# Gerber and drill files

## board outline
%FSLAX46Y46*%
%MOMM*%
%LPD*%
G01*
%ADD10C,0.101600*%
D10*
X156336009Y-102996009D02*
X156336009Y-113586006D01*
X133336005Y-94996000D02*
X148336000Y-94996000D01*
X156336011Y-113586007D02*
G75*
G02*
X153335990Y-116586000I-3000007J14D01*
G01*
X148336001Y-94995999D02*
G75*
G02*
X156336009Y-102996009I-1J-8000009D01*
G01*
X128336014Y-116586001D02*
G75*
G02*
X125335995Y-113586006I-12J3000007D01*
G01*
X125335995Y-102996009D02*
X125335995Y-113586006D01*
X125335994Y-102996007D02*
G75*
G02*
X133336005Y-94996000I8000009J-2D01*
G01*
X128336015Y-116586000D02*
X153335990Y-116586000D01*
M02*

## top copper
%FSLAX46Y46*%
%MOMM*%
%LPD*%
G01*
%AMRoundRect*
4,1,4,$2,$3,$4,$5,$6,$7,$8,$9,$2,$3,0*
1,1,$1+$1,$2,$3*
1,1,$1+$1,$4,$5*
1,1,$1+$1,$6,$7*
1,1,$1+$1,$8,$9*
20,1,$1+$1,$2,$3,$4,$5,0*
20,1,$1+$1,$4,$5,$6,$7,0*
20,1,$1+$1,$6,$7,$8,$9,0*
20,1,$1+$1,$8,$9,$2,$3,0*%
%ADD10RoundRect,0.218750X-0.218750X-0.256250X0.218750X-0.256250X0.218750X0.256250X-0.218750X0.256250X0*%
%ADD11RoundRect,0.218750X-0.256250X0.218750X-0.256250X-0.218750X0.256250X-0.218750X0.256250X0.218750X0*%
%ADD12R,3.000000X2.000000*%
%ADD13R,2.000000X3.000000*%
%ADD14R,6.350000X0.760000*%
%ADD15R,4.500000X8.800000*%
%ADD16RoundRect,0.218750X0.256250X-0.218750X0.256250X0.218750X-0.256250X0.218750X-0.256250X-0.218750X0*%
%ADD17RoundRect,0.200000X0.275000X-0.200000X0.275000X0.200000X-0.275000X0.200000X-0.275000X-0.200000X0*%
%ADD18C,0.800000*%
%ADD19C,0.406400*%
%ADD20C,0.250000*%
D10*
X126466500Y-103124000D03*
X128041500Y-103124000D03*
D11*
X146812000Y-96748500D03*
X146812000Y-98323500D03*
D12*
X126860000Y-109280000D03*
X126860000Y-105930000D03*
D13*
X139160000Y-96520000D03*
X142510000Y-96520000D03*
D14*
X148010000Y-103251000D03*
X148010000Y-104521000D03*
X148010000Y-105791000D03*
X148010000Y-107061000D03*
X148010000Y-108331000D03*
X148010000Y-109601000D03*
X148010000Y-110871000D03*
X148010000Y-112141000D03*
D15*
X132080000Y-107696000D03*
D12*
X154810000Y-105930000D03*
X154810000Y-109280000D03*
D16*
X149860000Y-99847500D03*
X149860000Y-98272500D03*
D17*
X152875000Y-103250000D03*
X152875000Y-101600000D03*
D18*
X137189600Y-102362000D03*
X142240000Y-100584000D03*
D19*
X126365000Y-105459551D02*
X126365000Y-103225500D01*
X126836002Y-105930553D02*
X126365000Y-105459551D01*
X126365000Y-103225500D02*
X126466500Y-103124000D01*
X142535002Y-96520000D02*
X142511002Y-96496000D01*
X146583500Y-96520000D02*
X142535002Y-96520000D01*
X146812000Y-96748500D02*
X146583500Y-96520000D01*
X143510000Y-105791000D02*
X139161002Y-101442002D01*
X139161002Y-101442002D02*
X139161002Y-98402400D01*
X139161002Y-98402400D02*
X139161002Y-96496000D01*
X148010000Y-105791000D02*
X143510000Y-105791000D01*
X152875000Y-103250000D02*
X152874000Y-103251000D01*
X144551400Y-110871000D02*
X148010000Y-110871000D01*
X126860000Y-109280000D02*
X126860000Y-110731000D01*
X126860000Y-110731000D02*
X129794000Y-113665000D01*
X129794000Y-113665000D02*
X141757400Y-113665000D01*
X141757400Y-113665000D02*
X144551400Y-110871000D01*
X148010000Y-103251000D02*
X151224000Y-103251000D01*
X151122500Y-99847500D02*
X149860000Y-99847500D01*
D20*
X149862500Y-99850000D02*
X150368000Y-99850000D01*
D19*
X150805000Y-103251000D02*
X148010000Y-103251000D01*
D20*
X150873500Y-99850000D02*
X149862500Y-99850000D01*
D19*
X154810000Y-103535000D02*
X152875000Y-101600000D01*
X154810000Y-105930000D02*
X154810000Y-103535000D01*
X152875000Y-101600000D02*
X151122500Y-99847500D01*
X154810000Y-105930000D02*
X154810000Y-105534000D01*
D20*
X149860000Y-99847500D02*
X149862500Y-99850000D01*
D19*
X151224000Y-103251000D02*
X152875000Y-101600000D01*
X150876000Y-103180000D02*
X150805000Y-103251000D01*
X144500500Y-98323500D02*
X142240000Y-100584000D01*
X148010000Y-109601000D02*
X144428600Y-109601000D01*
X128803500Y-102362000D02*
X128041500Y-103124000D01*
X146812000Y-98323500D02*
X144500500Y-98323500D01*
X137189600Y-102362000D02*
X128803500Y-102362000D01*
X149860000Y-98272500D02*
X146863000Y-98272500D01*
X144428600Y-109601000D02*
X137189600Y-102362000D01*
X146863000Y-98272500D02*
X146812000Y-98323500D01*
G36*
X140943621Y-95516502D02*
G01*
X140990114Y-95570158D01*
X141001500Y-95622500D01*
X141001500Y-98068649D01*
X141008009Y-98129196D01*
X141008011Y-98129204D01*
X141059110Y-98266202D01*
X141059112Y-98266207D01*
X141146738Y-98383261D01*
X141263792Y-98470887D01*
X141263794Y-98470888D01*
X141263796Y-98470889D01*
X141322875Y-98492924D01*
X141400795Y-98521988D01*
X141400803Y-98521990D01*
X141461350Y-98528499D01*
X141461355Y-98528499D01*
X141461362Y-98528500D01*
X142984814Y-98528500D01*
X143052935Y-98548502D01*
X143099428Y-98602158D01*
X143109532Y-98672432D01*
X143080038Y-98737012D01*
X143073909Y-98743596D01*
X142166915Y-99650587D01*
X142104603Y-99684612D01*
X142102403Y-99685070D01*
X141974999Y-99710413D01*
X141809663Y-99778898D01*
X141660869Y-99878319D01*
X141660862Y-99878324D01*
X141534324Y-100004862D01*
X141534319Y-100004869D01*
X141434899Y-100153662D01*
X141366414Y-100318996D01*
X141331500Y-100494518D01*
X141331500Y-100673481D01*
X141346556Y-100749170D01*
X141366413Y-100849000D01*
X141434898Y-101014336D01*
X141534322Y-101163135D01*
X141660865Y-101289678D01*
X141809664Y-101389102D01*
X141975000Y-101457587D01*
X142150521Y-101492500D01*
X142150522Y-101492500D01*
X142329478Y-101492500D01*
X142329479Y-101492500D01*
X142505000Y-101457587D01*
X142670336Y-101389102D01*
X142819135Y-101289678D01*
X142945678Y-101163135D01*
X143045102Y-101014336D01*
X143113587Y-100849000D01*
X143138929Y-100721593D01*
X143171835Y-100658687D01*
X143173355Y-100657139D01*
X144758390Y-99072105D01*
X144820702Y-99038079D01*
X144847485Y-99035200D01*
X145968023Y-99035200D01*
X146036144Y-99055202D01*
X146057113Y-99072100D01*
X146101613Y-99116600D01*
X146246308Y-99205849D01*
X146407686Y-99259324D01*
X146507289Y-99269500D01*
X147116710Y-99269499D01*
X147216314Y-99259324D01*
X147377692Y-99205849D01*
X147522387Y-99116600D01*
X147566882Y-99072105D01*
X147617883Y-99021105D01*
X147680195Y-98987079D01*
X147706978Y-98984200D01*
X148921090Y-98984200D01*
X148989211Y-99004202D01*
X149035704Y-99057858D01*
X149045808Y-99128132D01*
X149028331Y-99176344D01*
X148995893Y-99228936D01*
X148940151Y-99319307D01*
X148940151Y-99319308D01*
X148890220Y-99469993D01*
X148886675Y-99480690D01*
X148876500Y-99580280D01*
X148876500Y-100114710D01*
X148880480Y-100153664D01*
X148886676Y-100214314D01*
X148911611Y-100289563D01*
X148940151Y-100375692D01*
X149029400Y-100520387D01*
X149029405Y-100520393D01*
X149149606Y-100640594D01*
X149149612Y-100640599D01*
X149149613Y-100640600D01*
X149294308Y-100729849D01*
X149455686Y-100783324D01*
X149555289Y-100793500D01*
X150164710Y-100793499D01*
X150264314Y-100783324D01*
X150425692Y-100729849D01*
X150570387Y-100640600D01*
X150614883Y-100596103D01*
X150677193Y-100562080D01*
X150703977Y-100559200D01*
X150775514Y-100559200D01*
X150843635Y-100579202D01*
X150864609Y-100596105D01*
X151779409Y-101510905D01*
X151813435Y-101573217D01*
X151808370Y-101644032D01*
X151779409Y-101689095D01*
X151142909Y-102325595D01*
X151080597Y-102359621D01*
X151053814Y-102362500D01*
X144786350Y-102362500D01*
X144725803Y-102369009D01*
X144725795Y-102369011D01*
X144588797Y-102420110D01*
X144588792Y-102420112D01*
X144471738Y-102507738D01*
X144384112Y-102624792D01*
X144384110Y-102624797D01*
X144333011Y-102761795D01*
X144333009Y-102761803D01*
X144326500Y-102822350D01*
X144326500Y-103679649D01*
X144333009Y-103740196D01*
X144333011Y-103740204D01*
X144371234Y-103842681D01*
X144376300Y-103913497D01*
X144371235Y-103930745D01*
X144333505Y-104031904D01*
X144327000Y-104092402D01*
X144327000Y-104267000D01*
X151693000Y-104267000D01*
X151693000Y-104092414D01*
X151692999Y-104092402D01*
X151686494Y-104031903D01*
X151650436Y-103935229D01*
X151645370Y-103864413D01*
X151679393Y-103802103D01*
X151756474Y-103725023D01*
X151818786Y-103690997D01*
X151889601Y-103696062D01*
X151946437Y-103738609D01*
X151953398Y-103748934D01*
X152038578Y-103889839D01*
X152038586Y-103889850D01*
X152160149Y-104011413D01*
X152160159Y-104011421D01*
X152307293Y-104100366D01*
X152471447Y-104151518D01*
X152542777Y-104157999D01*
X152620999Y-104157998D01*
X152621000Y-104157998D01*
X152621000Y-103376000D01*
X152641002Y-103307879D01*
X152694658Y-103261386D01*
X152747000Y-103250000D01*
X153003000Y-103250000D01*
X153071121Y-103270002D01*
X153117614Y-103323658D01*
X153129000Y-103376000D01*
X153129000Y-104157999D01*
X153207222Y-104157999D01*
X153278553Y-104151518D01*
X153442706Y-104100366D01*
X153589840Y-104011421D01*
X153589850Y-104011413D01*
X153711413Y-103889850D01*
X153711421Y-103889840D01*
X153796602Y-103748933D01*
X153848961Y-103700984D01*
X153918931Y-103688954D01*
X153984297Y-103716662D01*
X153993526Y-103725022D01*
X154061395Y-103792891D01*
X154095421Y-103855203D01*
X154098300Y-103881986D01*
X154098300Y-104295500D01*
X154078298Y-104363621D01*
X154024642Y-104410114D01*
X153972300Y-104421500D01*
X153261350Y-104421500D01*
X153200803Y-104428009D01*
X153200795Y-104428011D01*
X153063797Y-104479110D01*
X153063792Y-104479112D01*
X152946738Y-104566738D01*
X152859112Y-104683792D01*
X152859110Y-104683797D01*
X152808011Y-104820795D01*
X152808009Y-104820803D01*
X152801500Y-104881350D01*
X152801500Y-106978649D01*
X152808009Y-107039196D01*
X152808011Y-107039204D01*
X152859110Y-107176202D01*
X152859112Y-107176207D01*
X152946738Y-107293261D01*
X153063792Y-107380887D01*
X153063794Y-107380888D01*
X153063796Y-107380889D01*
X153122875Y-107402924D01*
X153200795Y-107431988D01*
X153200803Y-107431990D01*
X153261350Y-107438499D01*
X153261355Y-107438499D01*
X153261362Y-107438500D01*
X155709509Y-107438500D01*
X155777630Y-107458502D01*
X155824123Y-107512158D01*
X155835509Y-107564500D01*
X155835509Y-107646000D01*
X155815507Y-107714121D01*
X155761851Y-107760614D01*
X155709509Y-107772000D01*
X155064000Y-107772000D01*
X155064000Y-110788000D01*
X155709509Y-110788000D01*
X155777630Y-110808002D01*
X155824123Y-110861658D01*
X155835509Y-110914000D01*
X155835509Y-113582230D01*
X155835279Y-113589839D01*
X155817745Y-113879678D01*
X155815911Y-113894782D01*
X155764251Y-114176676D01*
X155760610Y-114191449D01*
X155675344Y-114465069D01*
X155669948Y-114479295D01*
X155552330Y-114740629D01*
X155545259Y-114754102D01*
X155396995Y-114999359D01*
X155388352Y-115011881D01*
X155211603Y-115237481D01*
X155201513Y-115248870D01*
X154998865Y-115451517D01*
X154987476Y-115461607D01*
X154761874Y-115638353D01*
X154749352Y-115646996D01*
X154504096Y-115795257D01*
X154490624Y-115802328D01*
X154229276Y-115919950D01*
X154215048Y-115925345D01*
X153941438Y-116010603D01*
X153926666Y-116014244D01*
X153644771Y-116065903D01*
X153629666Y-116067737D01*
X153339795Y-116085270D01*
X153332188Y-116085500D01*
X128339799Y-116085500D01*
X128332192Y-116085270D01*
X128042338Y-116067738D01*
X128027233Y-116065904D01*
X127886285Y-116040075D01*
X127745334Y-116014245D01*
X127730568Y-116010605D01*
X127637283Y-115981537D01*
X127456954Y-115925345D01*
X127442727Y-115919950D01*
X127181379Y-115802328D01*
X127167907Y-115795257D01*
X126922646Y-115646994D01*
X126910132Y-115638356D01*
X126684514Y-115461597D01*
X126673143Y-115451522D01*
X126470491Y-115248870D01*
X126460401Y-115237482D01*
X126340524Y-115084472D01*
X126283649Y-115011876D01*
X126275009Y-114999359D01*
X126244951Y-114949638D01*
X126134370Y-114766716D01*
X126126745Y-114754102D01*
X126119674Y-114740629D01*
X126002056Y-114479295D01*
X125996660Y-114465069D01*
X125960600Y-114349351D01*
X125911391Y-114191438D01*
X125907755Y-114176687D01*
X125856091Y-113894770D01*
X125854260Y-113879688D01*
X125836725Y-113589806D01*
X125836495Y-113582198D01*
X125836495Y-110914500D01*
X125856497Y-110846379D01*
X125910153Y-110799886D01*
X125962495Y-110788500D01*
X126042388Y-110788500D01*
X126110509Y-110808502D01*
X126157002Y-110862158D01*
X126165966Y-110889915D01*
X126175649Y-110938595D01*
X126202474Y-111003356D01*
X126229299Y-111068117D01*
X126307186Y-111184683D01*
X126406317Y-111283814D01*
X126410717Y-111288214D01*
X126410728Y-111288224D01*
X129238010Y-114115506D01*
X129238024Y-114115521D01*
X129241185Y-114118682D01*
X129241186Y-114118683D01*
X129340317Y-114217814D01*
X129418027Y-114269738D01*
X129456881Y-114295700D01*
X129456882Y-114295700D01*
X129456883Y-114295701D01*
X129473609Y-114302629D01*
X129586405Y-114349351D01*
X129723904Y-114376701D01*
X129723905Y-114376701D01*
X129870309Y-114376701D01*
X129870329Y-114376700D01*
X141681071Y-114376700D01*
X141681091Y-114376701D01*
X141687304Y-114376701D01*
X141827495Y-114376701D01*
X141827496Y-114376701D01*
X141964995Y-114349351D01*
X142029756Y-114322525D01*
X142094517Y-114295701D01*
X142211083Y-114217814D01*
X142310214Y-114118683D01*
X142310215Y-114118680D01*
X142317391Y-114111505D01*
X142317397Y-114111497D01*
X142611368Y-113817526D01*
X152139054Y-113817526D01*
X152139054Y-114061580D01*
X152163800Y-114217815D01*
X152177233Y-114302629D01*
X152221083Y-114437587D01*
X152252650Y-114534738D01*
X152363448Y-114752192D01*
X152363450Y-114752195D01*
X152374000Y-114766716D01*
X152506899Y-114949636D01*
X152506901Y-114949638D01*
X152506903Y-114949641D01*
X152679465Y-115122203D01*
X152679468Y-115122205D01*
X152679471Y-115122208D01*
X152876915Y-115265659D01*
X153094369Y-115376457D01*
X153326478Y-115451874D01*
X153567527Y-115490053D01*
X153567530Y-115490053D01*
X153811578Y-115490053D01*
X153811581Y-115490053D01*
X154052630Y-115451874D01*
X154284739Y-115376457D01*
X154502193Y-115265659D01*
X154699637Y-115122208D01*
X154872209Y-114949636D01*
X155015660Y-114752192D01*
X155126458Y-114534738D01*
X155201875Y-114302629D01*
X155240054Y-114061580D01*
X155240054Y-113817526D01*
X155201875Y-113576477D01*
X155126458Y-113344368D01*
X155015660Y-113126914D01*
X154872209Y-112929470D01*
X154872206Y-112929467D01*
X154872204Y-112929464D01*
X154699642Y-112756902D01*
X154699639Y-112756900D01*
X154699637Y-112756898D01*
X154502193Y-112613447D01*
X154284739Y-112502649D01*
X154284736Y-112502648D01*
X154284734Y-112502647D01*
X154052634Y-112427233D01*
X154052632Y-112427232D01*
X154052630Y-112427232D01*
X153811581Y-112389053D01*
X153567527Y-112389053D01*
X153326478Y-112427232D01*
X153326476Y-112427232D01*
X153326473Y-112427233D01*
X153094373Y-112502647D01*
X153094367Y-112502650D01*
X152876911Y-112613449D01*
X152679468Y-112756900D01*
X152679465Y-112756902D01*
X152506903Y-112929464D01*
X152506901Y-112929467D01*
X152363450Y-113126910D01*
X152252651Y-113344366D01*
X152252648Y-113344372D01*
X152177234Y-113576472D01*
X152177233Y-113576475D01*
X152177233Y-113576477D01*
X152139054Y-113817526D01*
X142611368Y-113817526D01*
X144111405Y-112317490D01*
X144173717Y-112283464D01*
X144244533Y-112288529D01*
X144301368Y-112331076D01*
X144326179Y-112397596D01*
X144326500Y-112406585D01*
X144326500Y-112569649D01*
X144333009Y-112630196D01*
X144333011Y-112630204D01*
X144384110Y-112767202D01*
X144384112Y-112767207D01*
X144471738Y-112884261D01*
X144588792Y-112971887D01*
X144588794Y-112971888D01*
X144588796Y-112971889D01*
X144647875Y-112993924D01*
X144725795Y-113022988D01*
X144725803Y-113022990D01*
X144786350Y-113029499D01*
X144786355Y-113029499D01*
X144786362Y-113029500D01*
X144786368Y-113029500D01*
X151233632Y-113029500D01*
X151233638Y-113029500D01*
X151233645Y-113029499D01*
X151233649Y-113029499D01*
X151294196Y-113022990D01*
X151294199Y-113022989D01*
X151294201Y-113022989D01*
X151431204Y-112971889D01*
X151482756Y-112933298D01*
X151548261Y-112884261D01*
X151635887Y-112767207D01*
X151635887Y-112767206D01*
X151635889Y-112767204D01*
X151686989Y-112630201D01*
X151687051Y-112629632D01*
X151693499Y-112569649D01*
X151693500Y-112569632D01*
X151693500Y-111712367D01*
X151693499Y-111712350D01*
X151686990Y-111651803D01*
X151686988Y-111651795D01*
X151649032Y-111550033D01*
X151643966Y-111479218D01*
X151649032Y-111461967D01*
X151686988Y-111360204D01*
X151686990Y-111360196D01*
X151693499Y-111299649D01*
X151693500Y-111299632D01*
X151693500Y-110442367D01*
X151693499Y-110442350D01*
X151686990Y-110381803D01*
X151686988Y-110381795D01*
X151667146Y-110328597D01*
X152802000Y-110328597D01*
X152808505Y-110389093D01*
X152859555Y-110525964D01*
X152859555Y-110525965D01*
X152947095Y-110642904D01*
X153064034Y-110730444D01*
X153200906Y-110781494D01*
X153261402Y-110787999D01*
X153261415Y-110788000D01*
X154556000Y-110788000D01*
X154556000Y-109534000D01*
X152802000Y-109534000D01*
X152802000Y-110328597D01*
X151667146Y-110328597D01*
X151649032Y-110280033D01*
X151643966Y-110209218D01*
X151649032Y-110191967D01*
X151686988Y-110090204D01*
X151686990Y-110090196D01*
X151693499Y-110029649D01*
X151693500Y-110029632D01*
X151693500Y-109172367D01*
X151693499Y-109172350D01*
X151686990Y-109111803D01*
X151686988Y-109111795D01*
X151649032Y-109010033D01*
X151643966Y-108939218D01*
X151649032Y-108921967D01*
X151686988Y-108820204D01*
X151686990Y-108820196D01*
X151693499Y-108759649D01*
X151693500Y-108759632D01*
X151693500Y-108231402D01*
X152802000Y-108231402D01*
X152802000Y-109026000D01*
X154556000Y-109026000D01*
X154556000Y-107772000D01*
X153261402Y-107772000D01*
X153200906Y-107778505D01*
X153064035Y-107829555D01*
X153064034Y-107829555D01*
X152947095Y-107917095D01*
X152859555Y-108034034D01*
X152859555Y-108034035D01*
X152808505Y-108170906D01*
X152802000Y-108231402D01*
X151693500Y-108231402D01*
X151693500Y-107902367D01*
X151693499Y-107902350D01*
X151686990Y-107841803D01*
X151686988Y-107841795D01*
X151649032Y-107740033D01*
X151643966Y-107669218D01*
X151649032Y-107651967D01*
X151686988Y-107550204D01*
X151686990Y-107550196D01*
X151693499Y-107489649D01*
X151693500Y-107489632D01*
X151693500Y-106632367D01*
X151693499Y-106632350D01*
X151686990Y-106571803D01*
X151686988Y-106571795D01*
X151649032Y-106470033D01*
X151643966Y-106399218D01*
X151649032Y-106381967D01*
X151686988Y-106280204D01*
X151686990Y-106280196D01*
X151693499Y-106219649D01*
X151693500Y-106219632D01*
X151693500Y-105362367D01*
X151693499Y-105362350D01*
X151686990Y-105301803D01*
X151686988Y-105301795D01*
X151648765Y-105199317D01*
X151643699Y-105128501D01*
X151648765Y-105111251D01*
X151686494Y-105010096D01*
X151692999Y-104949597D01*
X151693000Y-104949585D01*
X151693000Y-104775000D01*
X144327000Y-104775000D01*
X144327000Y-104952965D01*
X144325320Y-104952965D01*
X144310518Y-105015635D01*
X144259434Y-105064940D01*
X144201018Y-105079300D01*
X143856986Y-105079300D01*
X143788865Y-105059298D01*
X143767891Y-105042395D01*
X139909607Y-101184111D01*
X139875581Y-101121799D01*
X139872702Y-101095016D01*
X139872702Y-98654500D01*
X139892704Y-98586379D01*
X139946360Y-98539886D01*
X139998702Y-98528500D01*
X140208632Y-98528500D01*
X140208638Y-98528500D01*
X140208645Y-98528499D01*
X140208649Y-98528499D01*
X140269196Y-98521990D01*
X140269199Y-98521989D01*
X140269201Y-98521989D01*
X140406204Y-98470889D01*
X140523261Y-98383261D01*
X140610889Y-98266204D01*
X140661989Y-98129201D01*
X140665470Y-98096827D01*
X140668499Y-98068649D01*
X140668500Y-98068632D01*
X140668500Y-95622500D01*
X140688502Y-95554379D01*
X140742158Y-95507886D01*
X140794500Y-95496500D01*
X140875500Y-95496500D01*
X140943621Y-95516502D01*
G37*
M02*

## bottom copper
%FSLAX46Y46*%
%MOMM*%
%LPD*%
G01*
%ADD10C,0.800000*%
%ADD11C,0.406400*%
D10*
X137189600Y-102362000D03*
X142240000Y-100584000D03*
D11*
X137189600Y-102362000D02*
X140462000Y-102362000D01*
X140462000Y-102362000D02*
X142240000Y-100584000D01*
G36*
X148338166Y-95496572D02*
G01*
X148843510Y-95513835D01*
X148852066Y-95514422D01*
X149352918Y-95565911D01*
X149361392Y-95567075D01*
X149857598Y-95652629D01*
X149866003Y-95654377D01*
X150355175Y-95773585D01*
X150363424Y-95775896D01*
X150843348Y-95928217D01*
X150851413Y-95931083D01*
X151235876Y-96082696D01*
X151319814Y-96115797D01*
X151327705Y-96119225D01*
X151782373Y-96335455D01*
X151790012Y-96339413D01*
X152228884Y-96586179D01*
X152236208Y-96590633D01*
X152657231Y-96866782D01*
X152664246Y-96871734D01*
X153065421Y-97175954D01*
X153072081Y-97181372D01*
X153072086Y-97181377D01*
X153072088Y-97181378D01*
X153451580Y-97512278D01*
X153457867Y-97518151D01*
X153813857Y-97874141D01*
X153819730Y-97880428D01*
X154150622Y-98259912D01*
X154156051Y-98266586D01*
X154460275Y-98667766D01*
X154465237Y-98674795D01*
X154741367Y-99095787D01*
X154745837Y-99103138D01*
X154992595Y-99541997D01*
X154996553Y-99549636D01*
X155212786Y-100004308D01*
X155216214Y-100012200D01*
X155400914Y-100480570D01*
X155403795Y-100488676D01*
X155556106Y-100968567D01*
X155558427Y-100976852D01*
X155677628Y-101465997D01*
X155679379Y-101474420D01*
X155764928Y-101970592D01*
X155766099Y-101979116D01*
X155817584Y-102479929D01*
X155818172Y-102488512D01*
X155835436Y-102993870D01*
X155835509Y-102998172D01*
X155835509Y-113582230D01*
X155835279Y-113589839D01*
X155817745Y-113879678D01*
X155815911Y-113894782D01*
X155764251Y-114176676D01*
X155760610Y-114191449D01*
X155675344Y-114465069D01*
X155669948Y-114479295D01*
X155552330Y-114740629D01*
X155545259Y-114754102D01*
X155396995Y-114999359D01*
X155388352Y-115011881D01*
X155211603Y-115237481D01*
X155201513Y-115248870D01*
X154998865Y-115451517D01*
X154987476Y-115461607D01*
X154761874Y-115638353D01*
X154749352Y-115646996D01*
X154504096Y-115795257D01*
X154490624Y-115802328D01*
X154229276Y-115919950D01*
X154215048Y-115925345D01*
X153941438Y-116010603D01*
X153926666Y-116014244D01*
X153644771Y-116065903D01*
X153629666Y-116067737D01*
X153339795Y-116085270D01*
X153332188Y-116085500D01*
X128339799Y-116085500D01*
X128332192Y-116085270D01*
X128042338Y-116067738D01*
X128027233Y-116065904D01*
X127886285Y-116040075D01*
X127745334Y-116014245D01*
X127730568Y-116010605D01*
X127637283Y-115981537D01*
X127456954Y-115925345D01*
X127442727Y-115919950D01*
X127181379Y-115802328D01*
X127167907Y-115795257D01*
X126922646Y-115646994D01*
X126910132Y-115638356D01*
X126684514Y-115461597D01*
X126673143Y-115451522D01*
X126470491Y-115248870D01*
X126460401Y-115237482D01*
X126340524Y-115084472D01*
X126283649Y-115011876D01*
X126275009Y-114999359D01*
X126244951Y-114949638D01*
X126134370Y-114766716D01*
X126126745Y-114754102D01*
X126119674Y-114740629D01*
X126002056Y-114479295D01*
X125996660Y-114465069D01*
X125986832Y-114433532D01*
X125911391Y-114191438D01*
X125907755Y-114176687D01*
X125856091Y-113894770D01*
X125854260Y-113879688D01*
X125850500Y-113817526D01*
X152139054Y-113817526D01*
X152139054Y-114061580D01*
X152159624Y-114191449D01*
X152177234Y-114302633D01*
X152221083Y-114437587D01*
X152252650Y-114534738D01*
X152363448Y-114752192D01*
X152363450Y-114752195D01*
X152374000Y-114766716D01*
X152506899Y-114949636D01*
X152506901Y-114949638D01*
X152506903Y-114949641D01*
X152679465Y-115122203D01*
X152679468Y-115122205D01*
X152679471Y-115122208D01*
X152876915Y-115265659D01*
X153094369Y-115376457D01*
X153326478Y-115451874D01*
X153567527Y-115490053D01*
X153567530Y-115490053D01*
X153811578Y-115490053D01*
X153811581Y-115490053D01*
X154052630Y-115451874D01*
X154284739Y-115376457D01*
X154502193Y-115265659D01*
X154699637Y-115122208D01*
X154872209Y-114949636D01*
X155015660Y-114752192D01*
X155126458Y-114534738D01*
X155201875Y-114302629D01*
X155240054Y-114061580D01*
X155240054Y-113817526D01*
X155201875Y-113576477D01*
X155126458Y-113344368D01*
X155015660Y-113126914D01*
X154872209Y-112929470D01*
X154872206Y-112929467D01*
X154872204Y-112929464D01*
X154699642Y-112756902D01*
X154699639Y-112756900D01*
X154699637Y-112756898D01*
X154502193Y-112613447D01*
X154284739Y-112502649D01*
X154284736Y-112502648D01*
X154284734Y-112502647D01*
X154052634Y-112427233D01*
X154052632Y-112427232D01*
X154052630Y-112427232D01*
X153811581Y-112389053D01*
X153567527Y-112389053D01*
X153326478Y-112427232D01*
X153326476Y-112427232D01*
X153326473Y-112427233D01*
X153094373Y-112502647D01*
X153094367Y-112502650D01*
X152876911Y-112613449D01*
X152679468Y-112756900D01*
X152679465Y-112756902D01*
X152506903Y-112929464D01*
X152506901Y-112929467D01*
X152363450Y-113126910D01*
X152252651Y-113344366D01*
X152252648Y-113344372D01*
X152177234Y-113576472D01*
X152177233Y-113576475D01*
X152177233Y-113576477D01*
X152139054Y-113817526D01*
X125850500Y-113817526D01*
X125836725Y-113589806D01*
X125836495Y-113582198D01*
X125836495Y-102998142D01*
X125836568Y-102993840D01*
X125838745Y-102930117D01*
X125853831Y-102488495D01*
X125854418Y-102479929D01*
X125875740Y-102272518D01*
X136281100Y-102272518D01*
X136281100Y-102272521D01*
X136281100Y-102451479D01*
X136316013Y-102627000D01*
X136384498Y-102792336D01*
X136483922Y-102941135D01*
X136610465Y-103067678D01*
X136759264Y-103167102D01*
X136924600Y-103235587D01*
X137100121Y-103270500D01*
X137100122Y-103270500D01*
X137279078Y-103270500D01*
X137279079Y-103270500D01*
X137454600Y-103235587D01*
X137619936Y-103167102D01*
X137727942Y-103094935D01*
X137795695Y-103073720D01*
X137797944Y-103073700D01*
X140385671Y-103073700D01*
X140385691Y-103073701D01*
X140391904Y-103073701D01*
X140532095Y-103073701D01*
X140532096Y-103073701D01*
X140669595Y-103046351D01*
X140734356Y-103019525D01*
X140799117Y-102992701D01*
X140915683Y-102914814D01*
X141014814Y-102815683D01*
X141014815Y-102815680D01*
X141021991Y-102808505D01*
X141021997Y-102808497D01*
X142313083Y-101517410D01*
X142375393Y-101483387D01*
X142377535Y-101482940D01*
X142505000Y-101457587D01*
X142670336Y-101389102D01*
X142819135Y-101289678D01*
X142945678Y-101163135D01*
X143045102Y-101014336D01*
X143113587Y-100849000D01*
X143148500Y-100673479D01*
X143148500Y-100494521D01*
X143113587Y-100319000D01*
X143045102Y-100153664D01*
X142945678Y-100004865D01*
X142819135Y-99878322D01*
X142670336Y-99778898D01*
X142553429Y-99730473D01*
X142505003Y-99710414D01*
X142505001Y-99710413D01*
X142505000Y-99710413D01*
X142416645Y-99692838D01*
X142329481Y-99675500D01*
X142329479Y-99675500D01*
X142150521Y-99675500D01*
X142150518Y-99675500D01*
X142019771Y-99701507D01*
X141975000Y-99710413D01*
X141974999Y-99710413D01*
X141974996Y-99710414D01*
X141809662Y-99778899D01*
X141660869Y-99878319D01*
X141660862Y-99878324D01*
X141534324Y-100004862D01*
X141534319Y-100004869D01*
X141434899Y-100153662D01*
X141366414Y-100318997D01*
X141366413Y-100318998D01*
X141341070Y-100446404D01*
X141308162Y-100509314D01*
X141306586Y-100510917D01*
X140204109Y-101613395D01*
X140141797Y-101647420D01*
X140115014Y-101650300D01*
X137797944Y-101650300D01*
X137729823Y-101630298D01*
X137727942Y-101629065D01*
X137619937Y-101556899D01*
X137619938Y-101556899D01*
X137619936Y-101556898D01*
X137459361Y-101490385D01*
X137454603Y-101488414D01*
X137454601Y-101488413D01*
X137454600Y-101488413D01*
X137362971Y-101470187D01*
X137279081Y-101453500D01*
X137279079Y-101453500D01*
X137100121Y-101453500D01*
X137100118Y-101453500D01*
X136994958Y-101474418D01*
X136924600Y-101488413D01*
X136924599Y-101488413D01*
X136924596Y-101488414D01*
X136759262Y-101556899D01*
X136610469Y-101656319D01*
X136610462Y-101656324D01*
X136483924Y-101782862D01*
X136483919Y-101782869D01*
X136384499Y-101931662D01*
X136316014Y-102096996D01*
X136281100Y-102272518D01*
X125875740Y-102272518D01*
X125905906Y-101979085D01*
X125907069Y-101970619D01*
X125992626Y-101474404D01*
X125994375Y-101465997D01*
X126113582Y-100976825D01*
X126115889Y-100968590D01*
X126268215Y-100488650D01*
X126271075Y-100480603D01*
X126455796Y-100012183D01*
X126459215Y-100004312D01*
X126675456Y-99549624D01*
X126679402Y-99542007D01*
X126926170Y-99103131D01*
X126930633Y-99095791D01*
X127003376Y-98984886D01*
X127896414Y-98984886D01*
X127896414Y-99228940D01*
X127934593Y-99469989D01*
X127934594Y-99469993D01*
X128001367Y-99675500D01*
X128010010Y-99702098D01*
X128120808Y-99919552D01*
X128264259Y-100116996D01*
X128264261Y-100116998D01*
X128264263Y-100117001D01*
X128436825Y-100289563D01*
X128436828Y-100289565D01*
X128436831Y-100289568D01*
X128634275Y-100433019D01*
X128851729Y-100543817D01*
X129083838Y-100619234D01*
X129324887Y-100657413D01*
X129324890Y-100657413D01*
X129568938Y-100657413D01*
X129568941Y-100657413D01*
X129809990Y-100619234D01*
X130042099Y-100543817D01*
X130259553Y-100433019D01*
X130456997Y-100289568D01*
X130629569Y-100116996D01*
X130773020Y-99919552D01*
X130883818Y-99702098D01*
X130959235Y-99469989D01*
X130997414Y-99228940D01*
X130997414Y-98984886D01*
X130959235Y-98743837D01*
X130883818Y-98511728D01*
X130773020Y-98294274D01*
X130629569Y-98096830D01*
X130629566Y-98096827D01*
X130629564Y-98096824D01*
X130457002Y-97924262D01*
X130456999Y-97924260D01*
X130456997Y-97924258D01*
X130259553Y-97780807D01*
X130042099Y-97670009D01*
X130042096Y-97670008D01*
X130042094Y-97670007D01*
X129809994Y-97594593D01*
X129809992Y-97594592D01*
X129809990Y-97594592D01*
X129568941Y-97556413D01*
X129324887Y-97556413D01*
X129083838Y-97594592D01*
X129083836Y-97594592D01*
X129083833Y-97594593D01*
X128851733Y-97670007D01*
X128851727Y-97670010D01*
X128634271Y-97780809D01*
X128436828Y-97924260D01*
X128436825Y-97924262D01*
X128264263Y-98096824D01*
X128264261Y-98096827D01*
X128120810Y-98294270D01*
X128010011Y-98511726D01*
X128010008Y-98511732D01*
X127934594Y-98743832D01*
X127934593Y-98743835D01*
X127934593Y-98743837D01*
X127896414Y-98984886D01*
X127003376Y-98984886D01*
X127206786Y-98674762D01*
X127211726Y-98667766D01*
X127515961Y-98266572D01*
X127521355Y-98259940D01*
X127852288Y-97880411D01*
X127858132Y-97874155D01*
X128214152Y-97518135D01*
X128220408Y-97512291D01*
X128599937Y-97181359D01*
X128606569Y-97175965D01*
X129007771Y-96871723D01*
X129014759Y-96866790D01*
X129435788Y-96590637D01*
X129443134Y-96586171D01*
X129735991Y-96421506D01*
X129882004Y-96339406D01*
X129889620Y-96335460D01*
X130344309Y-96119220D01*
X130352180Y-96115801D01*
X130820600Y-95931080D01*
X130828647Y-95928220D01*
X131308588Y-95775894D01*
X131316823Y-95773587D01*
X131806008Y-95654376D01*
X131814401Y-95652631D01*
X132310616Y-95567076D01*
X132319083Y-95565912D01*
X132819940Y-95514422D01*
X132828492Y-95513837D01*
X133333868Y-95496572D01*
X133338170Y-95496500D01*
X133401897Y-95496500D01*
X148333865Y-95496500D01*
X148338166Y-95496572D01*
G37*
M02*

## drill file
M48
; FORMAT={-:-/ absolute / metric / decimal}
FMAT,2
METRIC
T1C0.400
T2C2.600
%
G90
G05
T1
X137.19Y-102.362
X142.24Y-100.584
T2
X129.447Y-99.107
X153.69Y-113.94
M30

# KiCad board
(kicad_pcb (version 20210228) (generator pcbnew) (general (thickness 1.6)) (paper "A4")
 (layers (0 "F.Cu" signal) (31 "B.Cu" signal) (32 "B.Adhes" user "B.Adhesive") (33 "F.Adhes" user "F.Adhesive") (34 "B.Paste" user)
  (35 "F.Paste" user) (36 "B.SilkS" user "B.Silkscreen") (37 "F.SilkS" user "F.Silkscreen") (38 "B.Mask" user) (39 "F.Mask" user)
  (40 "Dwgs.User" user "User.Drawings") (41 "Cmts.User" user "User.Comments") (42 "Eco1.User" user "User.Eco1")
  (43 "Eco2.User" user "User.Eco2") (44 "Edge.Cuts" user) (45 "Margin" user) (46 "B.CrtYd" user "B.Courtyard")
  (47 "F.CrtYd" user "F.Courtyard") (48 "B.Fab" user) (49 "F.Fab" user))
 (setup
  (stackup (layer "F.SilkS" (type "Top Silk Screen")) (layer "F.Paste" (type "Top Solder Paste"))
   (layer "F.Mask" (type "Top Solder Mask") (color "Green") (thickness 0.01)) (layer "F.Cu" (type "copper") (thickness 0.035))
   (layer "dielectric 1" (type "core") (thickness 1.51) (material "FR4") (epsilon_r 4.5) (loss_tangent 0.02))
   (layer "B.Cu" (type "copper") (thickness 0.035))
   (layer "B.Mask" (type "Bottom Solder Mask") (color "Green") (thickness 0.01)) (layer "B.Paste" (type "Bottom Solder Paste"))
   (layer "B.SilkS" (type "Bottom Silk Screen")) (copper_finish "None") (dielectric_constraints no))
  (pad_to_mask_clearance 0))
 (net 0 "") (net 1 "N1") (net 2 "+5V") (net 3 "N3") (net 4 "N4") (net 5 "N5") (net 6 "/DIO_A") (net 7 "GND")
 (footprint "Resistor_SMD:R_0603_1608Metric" (layer "F.Cu") (at 127.254 103.124)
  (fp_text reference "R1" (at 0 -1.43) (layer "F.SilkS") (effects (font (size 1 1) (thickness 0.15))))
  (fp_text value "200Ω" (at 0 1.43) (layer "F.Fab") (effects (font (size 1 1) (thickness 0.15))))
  (pad "1" smd roundrect (at -0.7875 0) (locked) (size 0.875 0.95) (layers "F.Cu" "F.Paste" "F.Mask") (roundrect_rratio 0.25) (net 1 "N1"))
  (pad "2" smd roundrect (at 0.7875 0) (locked) (size 0.875 0.95) (layers "F.Cu" "F.Paste" "F.Mask") (roundrect_rratio 0.25) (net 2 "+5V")))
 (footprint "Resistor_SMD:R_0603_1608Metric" (layer "F.Cu") (at 146.812 97.536 -90)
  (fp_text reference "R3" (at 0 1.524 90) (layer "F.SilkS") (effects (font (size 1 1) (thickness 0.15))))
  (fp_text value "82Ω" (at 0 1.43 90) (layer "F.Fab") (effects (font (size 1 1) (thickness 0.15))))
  (pad "1" smd roundrect (at -0.7875 0 270) (locked) (size 0.875 0.95) (layers "F.Cu" "F.Paste" "F.Mask") (roundrect_rratio 0.25)
   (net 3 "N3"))
  (pad "2" smd roundrect (at 0.7875 0 270) (locked) (size 0.875 0.95) (layers "F.Cu" "F.Paste" "F.Mask") (roundrect_rratio 0.25)
   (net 2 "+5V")))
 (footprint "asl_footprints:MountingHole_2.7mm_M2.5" (layer "F.Cu") (at 129.446914 99.106913)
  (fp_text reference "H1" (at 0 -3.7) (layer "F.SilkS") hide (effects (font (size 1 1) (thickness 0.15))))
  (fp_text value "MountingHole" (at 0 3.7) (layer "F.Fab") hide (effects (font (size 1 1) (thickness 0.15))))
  (pad "" np_thru_hole circle (at 0 0) (locked) (size 2.6 2.6) (drill 2.6) (layers *.Cu *.Mask)))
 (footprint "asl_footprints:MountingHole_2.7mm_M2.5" (layer "F.Cu") (at 153.689554 113.939553)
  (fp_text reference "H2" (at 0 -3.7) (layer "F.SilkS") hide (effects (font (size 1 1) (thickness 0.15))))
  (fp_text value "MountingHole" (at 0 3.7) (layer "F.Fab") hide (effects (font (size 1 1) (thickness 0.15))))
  (pad "" np_thru_hole circle (at 0 0) (locked) (size 2.6 2.6) (drill 2.6) (layers *.Cu *.Mask)))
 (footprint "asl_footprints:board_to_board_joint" (layer "F.Cu") (at 128.36 107.605 90)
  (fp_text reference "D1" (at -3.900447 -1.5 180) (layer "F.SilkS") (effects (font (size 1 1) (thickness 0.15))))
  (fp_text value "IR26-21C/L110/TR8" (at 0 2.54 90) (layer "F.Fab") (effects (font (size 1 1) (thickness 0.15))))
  (pad "1" smd rect (at -1.675 -1.5 90) (locked) (size 2 3) (layers "F.Cu" "F.Paste" "F.Mask") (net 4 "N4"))
  (pad "2" smd rect (at 1.675 -1.5 90) (locked) (size 2 3) (layers "F.Cu" "F.Paste" "F.Mask") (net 1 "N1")))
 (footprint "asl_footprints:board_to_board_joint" (layer "F.Cu") (at 140.835 98.02)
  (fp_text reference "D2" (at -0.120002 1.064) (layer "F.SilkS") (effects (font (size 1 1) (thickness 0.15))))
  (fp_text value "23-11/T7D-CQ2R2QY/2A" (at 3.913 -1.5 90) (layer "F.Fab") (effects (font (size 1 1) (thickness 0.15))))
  (pad "1" smd rect (at -1.675 -1.5) (locked) (size 2 3) (layers "F.Cu" "F.Paste" "F.Mask") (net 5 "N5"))
  (pad "2" smd rect (at 1.675 -1.5) (locked) (size 2 3) (layers "F.Cu" "F.Paste" "F.Mask") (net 3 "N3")))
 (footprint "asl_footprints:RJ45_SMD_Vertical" (layer "F.Cu") (at 139.7 107.696 -90)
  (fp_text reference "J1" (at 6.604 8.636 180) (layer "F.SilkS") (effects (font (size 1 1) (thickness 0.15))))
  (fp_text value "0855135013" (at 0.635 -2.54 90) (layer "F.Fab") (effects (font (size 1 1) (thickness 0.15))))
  (pad "1" smd rect (at -4.445 -8.31) (locked) (size 6.35 0.76) (layers "F.Cu" "F.Paste" "F.Mask") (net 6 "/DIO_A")
   (solder_mask_margin 0.1016))
  (pad "2" smd rect (at -3.175 -8.31) (locked) (size 6.35 0.76) (layers "F.Cu" "F.Paste" "F.Mask") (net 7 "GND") (solder_mask_margin 0.1016))
  (pad "3" smd rect (at -1.905 -8.31) (locked) (size 6.35 0.76) (layers "F.Cu" "F.Paste" "F.Mask") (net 5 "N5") (solder_mask_margin 0.1016))
  (pad "4" smd rect (at -0.635 -8.31) (locked) (size 6.35 0.76) (layers "F.Cu" "F.Paste" "F.Mask") (solder_mask_margin 0.1016))
  (pad "5" smd rect (at 0.635 -8.31) (locked) (size 6.35 0.76) (layers "F.Cu" "F.Paste" "F.Mask") (solder_mask_margin 0.1016))
  (pad "6" smd rect (at 1.905 -8.31) (locked) (size 6.35 0.76) (layers "F.Cu" "F.Paste" "F.Mask") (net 2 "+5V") (solder_mask_margin 0.1016))
  (pad "7" smd rect (at 3.175 -8.31) (locked) (size 6.35 0.76) (layers "F.Cu" "F.Paste" "F.Mask") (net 4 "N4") (solder_mask_margin 0.1016))
  (pad "8" smd rect (at 4.445 -8.31) (locked) (size 6.35 0.76) (layers "F.Cu" "F.Paste" "F.Mask") (solder_mask_margin 0.1016))
  (pad "MNT" smd rect (at 0 7.62) (locked) (size 4.5 8.8) (layers "F.Cu" "F.Paste" "F.Mask") (solder_mask_margin 0.1016)))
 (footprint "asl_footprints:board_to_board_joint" (layer "F.Cu") (at 153.31 107.605 -90)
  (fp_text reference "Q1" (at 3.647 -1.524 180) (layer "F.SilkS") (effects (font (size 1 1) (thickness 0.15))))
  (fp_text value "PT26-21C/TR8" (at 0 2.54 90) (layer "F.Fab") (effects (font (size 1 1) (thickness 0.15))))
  (pad "1" smd rect (at -1.675 -1.5 270) (locked) (size 2 3) (layers "F.Cu" "F.Paste" "F.Mask") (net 6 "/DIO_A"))
  (pad "2" smd rect (at 1.675 -1.5 270) (locked) (size 2 3) (layers "F.Cu" "F.Paste" "F.Mask") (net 7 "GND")))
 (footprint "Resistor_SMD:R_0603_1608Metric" (layer "F.Cu") (at 149.86 99.06 90)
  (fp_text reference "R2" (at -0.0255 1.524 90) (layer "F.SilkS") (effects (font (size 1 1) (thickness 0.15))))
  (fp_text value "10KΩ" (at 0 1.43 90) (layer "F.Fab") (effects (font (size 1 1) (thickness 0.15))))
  (pad "1" smd roundrect (at -0.7875 0 90) (locked) (size 0.875 0.95) (layers "F.Cu" "F.Paste" "F.Mask") (roundrect_rratio 0.25)
   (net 6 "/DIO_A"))
  (pad "2" smd roundrect (at 0.7875 0 90) (locked) (size 0.875 0.95) (layers "F.Cu" "F.Paste" "F.Mask") (roundrect_rratio 0.25)
   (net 2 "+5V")))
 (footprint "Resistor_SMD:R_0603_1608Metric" (layer "F.Cu") (at 152.875 102.425 90)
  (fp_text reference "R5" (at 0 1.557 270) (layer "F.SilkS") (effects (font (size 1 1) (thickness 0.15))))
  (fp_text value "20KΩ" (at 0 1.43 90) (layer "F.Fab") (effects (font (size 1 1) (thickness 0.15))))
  (pad "1" smd roundrect (at -0.825 0 90) (locked) (size 0.8 0.95) (layers "F.Cu" "F.Paste" "F.Mask") (roundrect_rratio 0.25) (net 7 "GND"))
  (pad "2" smd roundrect (at 0.825 0 90) (locked) (size 0.8 0.95) (layers "F.Cu" "F.Paste" "F.Mask") (roundrect_rratio 0.25)
   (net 6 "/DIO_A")))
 (gr_line (start 156.336009 102.996009) (end 156.336009 113.586006) (layer "Edge.Cuts") (width 0.1016))
 (gr_line (start 133.336005 94.996) (end 148.336 94.996) (layer "Edge.Cuts") (width 0.1016))
 (gr_arc (start 153.336004 113.585993) (end 153.33599 116.586) (angle -90) (layer "Edge.Cuts") (width 0.1016))
 (gr_arc (start 148.336 102.996008) (end 156.336009 102.996009) (angle -90) (layer "Edge.Cuts") (width 0.1016))
 (gr_arc (start 128.336002 113.585994) (end 125.335995 113.586006) (angle -90) (layer "Edge.Cuts") (width 0.1016))
 (gr_line (start 125.335995 102.996009) (end 125.335995 113.586006) (layer "Edge.Cuts") (width 0.1016))
 (gr_arc (start 133.336003 102.996009) (end 133.336005 94.996) (angle -90) (layer "Edge.Cuts") (width 0.1016))
 (gr_line (start 128.336015 116.586) (end 153.33599 116.586) (layer "Edge.Cuts") (width 0.1016))
 (segment (start 126.365 105.459551) (end 126.365 103.2255) (width 0.4064) (layer "F.Cu") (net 1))
 (segment (start 126.836002 105.930553) (end 126.365 105.459551) (width 0.4064) (layer "F.Cu") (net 1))
 (segment (start 126.365 103.2255) (end 126.4665 103.124) (width 0.4064) (layer "F.Cu") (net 1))
 (segment (start 142.535002 96.52) (end 142.511002 96.496) (width 0.4064) (layer "F.Cu") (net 3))
 (segment (start 146.5835 96.52) (end 142.535002 96.52) (width 0.4064) (layer "F.Cu") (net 3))
 (segment (start 146.812 96.7485) (end 146.5835 96.52) (width 0.4064) (layer "F.Cu") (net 3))
 (segment (start 143.51 105.791) (end 139.161002 101.442002) (width 0.4064) (layer "F.Cu") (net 5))
 (segment (start 139.161002 101.442002) (end 139.161002 98.4024) (width 0.4064) (layer "F.Cu") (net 5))
 (segment (start 139.161002 98.4024) (end 139.161002 96.496) (width 0.4064) (layer "F.Cu") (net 5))
 (segment (start 148.01 105.791) (end 143.51 105.791) (width 0.4064) (layer "F.Cu") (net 5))
 (segment (start 152.875 103.25) (end 152.874 103.251) (width 0.4064) (layer "F.Cu") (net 7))
 (segment (start 144.5514 110.871) (end 148.01 110.871) (width 0.4064) (layer "F.Cu") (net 4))
 (segment (start 126.86 109.28) (end 126.86 110.731) (width 0.4064) (layer "F.Cu") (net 4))
 (segment (start 126.86 110.731) (end 129.794 113.665) (width 0.4064) (layer "F.Cu") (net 4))
 (segment (start 129.794 113.665) (end 141.7574 113.665) (width 0.4064) (layer "F.Cu") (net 4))
 (segment (start 141.7574 113.665) (end 144.5514 110.871) (width 0.4064) (layer "F.Cu") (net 4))
 (segment (start 148.01 103.251) (end 151.224 103.251) (width 0.4064) (layer "F.Cu") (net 6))
 (segment (start 151.1225 99.8475) (end 149.86 99.8475) (width 0.4064) (layer "F.Cu") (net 6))
 (segment (start 149.8625 99.85) (end 150.368 99.85) (width 0.25) (layer "F.Cu") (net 6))
 (segment (start 150.805 103.251) (end 148.01 103.251) (width 0.4064) (layer "F.Cu") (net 6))
 (segment (start 150.8735 99.85) (end 149.8625 99.85) (width 0.25) (layer "F.Cu") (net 6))
 (segment (start 154.81 103.535) (end 152.875 101.6) (width 0.4064) (layer "F.Cu") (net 6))
 (segment (start 154.81 105.93) (end 154.81 103.535) (width 0.4064) (layer "F.Cu") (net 6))
 (segment (start 152.875 101.6) (end 151.1225 99.8475) (width 0.4064) (layer "F.Cu") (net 6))
 (segment (start 154.81 105.93) (end 154.81 105.534) (width 0.4064) (layer "F.Cu") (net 6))
 (segment (start 149.86 99.8475) (end 149.8625 99.85) (width 0.25) (layer "F.Cu") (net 6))
 (segment (start 151.224 103.251) (end 152.875 101.6) (width 0.4064) (layer "F.Cu") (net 6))
 (segment (start 150.876 103.18) (end 150.805 103.251) (width 0.4064) (layer "F.Cu") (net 6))
 (segment (start 144.5005 98.3235) (end 142.24 100.584) (width 0.4064) (layer "F.Cu") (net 2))
 (segment (start 148.01 109.601) (end 144.4286 109.601) (width 0.4064) (layer "F.Cu") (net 2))
 (segment (start 128.8035 102.362) (end 128.0415 103.124) (width 0.4064) (layer "F.Cu") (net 2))
 (segment (start 146.812 98.3235) (end 144.5005 98.3235) (width 0.4064) (layer "F.Cu") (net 2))
 (segment (start 137.1896 102.362) (end 128.8035 102.362) (width 0.4064) (layer "F.Cu") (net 2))
 (segment (start 149.86 98.2725) (end 146.863 98.2725) (width 0.4064) (layer "F.Cu") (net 2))
 (segment (start 144.4286 109.601) (end 137.1896 102.362) (width 0.4064) (layer "F.Cu") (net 2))
 (segment (start 146.863 98.2725) (end 146.812 98.3235) (width 0.4064) (layer "F.Cu") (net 2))
 (via (at 137.1896 102.362) (size 0.8) (drill 0.4) (layers "F.Cu" "B.Cu") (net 2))
 (via (at 142.24 100.584) (size 0.8) (drill 0.4) (layers "F.Cu" "B.Cu") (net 2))
 (segment (start 137.1896 102.362) (end 140.462 102.362) (width 0.4064) (layer "B.Cu") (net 2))
 (segment (start 140.462 102.362) (end 142.24 100.584) (width 0.4064) (layer "B.Cu") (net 2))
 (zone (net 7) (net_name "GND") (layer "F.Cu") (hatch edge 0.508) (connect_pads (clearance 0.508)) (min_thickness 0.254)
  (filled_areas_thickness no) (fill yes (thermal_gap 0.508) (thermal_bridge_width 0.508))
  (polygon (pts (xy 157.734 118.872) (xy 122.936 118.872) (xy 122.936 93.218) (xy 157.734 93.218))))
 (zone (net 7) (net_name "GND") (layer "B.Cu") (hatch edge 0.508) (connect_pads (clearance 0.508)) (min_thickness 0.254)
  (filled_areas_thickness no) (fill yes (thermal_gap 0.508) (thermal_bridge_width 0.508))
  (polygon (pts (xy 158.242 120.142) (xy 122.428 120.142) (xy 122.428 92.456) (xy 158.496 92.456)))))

